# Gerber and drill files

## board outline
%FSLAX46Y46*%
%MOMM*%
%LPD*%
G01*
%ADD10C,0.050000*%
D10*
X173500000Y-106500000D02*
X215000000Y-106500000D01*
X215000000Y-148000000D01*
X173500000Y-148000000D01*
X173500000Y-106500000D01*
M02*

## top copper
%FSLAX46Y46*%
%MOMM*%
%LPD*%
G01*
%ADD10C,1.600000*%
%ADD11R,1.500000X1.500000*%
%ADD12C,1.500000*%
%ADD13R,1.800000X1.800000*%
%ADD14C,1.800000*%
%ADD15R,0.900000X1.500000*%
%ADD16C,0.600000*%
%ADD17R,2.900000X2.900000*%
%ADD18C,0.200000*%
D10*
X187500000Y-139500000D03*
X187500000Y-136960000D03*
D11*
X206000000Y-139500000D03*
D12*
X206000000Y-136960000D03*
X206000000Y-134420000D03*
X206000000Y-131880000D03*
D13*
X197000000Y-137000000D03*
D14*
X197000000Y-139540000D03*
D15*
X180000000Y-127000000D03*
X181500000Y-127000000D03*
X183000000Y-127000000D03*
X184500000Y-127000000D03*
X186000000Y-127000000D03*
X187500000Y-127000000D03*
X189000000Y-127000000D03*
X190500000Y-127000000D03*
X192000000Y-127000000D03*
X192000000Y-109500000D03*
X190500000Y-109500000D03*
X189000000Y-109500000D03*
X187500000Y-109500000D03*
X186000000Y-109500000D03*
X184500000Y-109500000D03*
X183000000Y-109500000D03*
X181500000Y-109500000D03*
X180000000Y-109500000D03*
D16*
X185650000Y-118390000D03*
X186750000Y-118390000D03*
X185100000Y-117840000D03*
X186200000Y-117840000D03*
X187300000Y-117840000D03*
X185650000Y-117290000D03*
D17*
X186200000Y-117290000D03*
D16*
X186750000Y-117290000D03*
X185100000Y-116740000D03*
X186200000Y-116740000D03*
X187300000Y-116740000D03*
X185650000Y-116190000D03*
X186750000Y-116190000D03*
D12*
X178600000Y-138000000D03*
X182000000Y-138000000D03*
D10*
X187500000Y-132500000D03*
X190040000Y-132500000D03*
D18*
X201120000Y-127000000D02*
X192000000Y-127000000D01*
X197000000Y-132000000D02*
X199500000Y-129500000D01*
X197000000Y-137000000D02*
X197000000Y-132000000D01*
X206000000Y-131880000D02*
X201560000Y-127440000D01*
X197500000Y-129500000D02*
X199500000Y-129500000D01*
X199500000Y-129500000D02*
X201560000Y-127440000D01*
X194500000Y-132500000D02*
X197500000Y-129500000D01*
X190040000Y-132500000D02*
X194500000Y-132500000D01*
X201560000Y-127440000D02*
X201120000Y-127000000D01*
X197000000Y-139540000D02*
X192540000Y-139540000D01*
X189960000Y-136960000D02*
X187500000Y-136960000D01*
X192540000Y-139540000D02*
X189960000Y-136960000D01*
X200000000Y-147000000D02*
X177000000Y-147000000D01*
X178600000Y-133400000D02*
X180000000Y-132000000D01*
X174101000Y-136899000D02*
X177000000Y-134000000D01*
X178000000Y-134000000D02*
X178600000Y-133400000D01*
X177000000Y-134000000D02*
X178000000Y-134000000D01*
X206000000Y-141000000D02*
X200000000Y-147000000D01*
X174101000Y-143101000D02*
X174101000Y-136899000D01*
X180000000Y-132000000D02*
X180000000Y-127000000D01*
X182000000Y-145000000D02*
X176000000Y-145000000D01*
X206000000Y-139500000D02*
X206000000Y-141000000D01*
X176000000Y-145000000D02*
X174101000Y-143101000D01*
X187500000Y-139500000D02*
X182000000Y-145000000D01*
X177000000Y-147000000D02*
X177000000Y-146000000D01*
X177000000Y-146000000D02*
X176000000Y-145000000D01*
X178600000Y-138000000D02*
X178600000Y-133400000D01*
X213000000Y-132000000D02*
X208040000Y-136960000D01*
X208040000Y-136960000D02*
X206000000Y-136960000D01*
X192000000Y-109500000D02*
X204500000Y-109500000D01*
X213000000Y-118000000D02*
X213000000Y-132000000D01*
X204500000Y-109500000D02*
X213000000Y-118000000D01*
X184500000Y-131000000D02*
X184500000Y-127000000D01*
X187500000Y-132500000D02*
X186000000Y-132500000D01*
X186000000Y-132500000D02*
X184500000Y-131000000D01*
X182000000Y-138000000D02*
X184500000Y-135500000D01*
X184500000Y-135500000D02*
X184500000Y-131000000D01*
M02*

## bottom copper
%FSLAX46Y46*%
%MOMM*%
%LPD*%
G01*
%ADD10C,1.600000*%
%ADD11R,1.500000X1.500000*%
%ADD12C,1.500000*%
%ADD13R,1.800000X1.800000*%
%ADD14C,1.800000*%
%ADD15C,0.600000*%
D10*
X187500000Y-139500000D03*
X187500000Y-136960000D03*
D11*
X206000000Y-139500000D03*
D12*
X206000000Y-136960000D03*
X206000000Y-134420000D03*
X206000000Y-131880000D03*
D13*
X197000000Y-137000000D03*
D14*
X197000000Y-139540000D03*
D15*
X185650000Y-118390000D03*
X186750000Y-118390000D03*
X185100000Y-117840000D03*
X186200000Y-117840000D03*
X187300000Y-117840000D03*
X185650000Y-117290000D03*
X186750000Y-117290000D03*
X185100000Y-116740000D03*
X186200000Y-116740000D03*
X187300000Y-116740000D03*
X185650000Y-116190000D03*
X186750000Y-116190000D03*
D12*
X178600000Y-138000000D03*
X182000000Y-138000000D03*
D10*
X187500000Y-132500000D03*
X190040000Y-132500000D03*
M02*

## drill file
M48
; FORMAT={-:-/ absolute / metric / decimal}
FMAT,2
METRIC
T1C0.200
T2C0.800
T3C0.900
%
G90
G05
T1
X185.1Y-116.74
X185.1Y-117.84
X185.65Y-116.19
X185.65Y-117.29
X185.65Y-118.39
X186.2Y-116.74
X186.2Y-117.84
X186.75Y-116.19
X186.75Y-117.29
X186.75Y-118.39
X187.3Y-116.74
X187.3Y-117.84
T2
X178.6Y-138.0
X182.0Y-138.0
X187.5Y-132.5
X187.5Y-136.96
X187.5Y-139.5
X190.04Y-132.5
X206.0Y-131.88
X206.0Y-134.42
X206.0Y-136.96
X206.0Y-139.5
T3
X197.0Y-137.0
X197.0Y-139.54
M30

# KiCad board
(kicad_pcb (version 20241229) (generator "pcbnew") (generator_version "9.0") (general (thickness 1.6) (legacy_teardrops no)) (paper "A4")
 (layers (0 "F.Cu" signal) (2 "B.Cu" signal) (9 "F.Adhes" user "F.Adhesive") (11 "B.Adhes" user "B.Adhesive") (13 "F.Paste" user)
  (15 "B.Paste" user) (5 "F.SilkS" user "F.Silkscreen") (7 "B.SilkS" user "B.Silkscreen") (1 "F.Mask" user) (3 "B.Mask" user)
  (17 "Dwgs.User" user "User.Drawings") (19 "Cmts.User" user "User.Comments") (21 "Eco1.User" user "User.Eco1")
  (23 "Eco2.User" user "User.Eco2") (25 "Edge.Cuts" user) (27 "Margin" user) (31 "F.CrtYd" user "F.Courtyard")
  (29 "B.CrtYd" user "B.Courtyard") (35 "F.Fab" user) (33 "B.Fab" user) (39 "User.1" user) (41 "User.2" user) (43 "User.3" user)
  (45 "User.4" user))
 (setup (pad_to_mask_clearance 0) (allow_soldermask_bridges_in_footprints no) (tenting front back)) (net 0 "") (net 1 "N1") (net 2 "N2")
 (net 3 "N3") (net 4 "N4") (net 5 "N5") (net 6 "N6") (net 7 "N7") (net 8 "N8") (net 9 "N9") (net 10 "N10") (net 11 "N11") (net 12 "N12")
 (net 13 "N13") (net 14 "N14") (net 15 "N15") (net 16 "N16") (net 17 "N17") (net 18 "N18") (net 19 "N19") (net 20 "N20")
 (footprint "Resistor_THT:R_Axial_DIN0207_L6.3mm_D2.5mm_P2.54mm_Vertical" (layer "F.Cu") (at 187.5 139.5 90)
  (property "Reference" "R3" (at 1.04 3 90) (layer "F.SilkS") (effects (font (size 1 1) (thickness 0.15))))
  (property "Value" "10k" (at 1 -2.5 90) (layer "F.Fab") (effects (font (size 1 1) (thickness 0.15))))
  (pad "1" thru_hole circle (at 0 0 90) (size 1.6 1.6) (drill 0.8) (layers "*.Cu" "*.Mask") (remove_unused_layers no) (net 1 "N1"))
  (pad "2" thru_hole circle (at 2.54 0 90) (size 1.6 1.6) (drill 0.8) (layers "*.Cu" "*.Mask") (remove_unused_layers no) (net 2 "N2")))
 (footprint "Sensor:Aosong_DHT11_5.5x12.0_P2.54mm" (layer "F.Cu") (at 206 139.5 180)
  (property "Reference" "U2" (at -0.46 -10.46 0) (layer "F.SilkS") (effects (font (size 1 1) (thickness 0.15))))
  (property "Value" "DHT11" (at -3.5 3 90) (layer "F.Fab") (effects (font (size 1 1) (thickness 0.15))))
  (pad "1" thru_hole rect (at 0 0 180) (size 1.5 1.5) (drill 0.8) (layers "*.Cu" "*.Mask") (remove_unused_layers no) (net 1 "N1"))
  (pad "2" thru_hole circle (at 0 2.54 180) (size 1.5 1.5) (drill 0.8) (layers "*.Cu" "*.Mask") (remove_unused_layers no) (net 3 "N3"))
  (pad "3" thru_hole circle (at 0 5.08 180) (size 1.5 1.5) (drill 0.8) (layers "*.Cu" "*.Mask") (remove_unused_layers no) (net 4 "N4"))
  (pad "4" thru_hole circle (at 0 7.62 180) (size 1.5 1.5) (drill 0.8) (layers "*.Cu" "*.Mask") (remove_unused_layers no) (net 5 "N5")))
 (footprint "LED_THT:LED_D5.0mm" (layer "F.Cu") (at 197 137 -90)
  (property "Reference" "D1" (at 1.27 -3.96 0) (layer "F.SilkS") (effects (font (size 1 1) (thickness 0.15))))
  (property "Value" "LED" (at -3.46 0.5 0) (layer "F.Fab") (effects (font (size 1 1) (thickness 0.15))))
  (pad "1" thru_hole rect (at 0 0 270) (size 1.8 1.8) (drill 0.9) (layers "*.Cu" "*.Mask") (remove_unused_layers no) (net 5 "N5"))
  (pad "2" thru_hole circle (at 2.54 0 270) (size 1.8 1.8) (drill 0.9) (layers "*.Cu" "*.Mask") (remove_unused_layers no) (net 2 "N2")))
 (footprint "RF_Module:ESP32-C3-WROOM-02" (layer "F.Cu") (at 186 118.25 90)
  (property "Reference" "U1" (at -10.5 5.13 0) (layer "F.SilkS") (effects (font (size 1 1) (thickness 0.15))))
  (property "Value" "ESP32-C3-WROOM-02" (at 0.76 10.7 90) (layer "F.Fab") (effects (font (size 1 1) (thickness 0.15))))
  (pad "" smd rect (at -0.14 -0.9 90) (size 0.7 0.7) (layers "F.Paste"))
  (pad "" smd rect (at -0.14 0.2 90) (size 0.7 0.7) (layers "F.Paste"))
  (pad "" smd rect (at -0.14 1.3 90) (size 0.7 0.7) (layers "F.Paste"))
  (pad "" smd rect (at 0.96 -0.9 90) (size 0.7 0.7) (layers "F.Paste"))
  (pad "" smd rect (at 0.96 0.2 90) (size 0.7 0.7) (layers "F.Paste"))
  (pad "" smd rect (at 0.96 1.3 90) (size 0.7 0.7) (layers "F.Paste"))
  (pad "" smd rect (at 2.06 -0.9 90) (size 0.7 0.7) (layers "F.Paste"))
  (pad "" smd rect (at 2.06 0.2 90) (size 0.7 0.7) (layers "F.Paste"))
  (pad "" smd rect (at 2.06 1.3 90) (size 0.7 0.7) (layers "F.Paste"))
  (pad "1" smd rect (at -8.75 -6 90) (size 1.5 0.9) (layers "F.Cu" "F.Mask" "F.Paste") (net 1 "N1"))
  (pad "2" smd rect (at -8.75 -4.5 90) (size 1.5 0.9) (layers "F.Cu" "F.Mask" "F.Paste") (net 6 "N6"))
  (pad "3" smd rect (at -8.75 -3 90) (size 1.5 0.9) (layers "F.Cu" "F.Mask" "F.Paste") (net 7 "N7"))
  (pad "4" smd rect (at -8.75 -1.5 90) (size 1.5 0.9) (layers "F.Cu" "F.Mask" "F.Paste") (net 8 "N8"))
  (pad "5" smd rect (at -8.75 0 90) (size 1.5 0.9) (layers "F.Cu" "F.Mask" "F.Paste") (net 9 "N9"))
  (pad "6" smd rect (at -8.75 1.5 90) (size 1.5 0.9) (layers "F.Cu" "F.Mask" "F.Paste") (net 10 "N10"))
  (pad "7" smd rect (at -8.75 3 90) (size 1.5 0.9) (layers "F.Cu" "F.Mask" "F.Paste") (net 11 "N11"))
  (pad "8" smd rect (at -8.75 4.5 90) (size 1.5 0.9) (layers "F.Cu" "F.Mask" "F.Paste") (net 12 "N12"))
  (pad "9" smd rect (at -8.75 6 90) (size 1.5 0.9) (layers "F.Cu" "F.Mask" "F.Paste") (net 5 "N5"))
  (pad "10" smd rect (at 8.75 6 90) (size 1.5 0.9) (layers "F.Cu" "F.Mask" "F.Paste") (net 3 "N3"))
  (pad "11" smd rect (at 8.75 4.5 90) (size 1.5 0.9) (layers "F.Cu" "F.Mask" "F.Paste") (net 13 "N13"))
  (pad "12" smd rect (at 8.75 3 90) (size 1.5 0.9) (layers "F.Cu" "F.Mask" "F.Paste") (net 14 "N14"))
  (pad "13" smd rect (at 8.75 1.5 90) (size 1.5 0.9) (layers "F.Cu" "F.Mask" "F.Paste") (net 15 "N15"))
  (pad "14" smd rect (at 8.75 0 90) (size 1.5 0.9) (layers "F.Cu" "F.Mask" "F.Paste") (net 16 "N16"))
  (pad "15" smd rect (at 8.75 -1.5 90) (size 1.5 0.9) (layers "F.Cu" "F.Mask" "F.Paste") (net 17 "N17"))
  (pad "16" smd rect (at 8.75 -3 90) (size 1.5 0.9) (layers "F.Cu" "F.Mask" "F.Paste") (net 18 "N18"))
  (pad "17" smd rect (at 8.75 -4.5 90) (size 1.5 0.9) (layers "F.Cu" "F.Mask" "F.Paste") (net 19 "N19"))
  (pad "18" smd rect (at 8.75 -6 90) (size 1.5 0.9) (layers "F.Cu" "F.Mask" "F.Paste") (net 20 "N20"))
  (pad "19" thru_hole circle (at -0.14 -0.35 90) (size 0.6 0.6) (drill 0.2) (layers "*.Cu" "F.Mask") (remove_unused_layers no) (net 5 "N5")
   (zone_connect 2))
  (pad "19" thru_hole circle (at -0.14 0.75 90) (size 0.6 0.6) (drill 0.2) (layers "*.Cu" "F.Mask") (remove_unused_layers no) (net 5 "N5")
   (zone_connect 2))
  (pad "19" thru_hole circle (at 0.41 -0.9 90) (size 0.6 0.6) (drill 0.2) (layers "*.Cu" "F.Mask") (remove_unused_layers no) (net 5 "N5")
   (zone_connect 2))
  (pad "19" thru_hole circle (at 0.41 0.2 90) (size 0.6 0.6) (drill 0.2) (layers "*.Cu" "F.Mask") (remove_unused_layers no) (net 5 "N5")
   (zone_connect 2))
  (pad "19" thru_hole circle (at 0.41 1.3 90) (size 0.6 0.6) (drill 0.2) (layers "*.Cu" "F.Mask") (remove_unused_layers no) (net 5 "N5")
   (zone_connect 2))
  (pad "19" thru_hole circle (at 0.96 -0.35 90) (size 0.6 0.6) (drill 0.2) (layers "*.Cu" "F.Mask") (remove_unused_layers no) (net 5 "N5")
   (zone_connect 2))
  (pad "19" smd rect (at 0.96 0.2 90) (size 2.9 2.9) (layers "F.Cu" "F.Mask") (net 5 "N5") (zone_connect 2))
  (pad "19" thru_hole circle (at 0.96 0.75 90) (size 0.6 0.6) (drill 0.2) (layers "*.Cu" "F.Mask") (remove_unused_layers no) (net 5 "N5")
   (zone_connect 2))
  (pad "19" thru_hole circle (at 1.51 -0.9 90) (size 0.6 0.6) (drill 0.2) (layers "*.Cu" "F.Mask") (remove_unused_layers no) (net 5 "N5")
   (zone_connect 2))
  (pad "19" thru_hole circle (at 1.51 0.2 90) (size 0.6 0.6) (drill 0.2) (layers "*.Cu" "F.Mask") (remove_unused_layers no) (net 5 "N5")
   (zone_connect 2))
  (pad "19" thru_hole circle (at 1.51 1.3 90) (size 0.6 0.6) (drill 0.2) (layers "*.Cu" "F.Mask") (remove_unused_layers no) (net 5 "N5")
   (zone_connect 2))
  (pad "19" thru_hole circle (at 2.06 -0.35 90) (size 0.6 0.6) (drill 0.2) (layers "*.Cu" "F.Mask") (remove_unused_layers no) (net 5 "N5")
   (zone_connect 2))
  (pad "19" thru_hole circle (at 2.06 0.75 90) (size 0.6 0.6) (drill 0.2) (layers "*.Cu" "F.Mask") (remove_unused_layers no) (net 5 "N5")
   (zone_connect 2))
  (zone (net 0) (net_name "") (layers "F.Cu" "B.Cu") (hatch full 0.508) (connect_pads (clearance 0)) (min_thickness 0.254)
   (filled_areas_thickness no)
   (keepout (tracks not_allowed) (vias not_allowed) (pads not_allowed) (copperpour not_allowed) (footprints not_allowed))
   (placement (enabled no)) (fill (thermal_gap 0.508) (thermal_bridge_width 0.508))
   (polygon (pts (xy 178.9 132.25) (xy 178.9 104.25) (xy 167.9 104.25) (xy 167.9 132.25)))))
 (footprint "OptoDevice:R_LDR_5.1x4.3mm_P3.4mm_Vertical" (layer "F.Cu") (at 178.6 138)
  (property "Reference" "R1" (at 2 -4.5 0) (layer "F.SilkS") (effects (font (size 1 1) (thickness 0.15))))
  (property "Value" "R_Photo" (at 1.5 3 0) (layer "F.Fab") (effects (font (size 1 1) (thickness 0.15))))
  (pad "1" thru_hole circle (at 0 0) (size 1.5 1.5) (drill 0.8) (layers "*.Cu" "*.Mask") (remove_unused_layers no) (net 1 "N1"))
  (pad "2" thru_hole circle (at 3.4 0) (size 1.5 1.5) (drill 0.8) (layers "*.Cu" "*.Mask") (remove_unused_layers no) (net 8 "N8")))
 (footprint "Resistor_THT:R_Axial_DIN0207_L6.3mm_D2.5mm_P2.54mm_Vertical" (layer "F.Cu") (at 187.5 132.5)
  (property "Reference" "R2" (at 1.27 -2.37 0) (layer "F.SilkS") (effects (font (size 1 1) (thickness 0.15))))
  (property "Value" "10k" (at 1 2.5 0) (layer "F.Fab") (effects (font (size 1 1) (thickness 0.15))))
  (pad "1" thru_hole circle (at 0 0) (size 1.6 1.6) (drill 0.8) (layers "*.Cu" "*.Mask") (remove_unused_layers no) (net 8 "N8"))
  (pad "2" thru_hole circle (at 2.54 0) (size 1.6 1.6) (drill 0.8) (layers "*.Cu" "*.Mask") (remove_unused_layers no) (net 5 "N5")))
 (gr_rect (start 173.5 106.5) (end 215 148) (stroke (width 0.05) (type default)) (fill no) (layer "Edge.Cuts"))
 (segment (start 201.12 127) (end 192 127) (width 0.2) (layer "F.Cu") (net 5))
 (segment (start 197 132) (end 199.5 129.5) (width 0.2) (layer "F.Cu") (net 5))
 (segment (start 197 137) (end 197 132) (width 0.2) (layer "F.Cu") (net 5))
 (segment (start 206 131.88) (end 201.56 127.44) (width 0.2) (layer "F.Cu") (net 5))
 (segment (start 197.5 129.5) (end 199.5 129.5) (width 0.2) (layer "F.Cu") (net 5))
 (segment (start 199.5 129.5) (end 201.56 127.44) (width 0.2) (layer "F.Cu") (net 5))
 (segment (start 194.5 132.5) (end 197.5 129.5) (width 0.2) (layer "F.Cu") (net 5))
 (segment (start 190.04 132.5) (end 194.5 132.5) (width 0.2) (layer "F.Cu") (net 5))
 (segment (start 201.56 127.44) (end 201.12 127) (width 0.2) (layer "F.Cu") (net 5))
 (segment (start 197 139.54) (end 192.54 139.54) (width 0.2) (layer "F.Cu") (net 2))
 (segment (start 189.96 136.96) (end 187.5 136.96) (width 0.2) (layer "F.Cu") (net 2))
 (segment (start 192.54 139.54) (end 189.96 136.96) (width 0.2) (layer "F.Cu") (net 2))
 (segment (start 200 147) (end 177 147) (width 0.2) (layer "F.Cu") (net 1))
 (segment (start 178.6 133.4) (end 180 132) (width 0.2) (layer "F.Cu") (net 1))
 (segment (start 174.101 136.899) (end 177 134) (width 0.2) (layer "F.Cu") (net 1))
 (segment (start 178 134) (end 178.6 133.4) (width 0.2) (layer "F.Cu") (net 1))
 (segment (start 177 134) (end 178 134) (width 0.2) (layer "F.Cu") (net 1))
 (segment (start 206 141) (end 200 147) (width 0.2) (layer "F.Cu") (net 1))
 (segment (start 174.101 143.101) (end 174.101 136.899) (width 0.2) (layer "F.Cu") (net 1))
 (segment (start 180 132) (end 180 127) (width 0.2) (layer "F.Cu") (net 1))
 (segment (start 182 145) (end 176 145) (width 0.2) (layer "F.Cu") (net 1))
 (segment (start 206 139.5) (end 206 141) (width 0.2) (layer "F.Cu") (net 1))
 (segment (start 176 145) (end 174.101 143.101) (width 0.2) (layer "F.Cu") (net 1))
 (segment (start 187.5 139.5) (end 182 145) (width 0.2) (layer "F.Cu") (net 1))
 (segment (start 177 147) (end 177 146) (width 0.2) (layer "F.Cu") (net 1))
 (segment (start 177 146) (end 176 145) (width 0.2) (layer "F.Cu") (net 1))
 (segment (start 178.6 138) (end 178.6 133.4) (width 0.2) (layer "F.Cu") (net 1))
 (segment (start 213 132) (end 208.04 136.96) (width 0.2) (layer "F.Cu") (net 3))
 (segment (start 208.04 136.96) (end 206 136.96) (width 0.2) (layer "F.Cu") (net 3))
 (segment (start 192 109.5) (end 204.5 109.5) (width 0.2) (layer "F.Cu") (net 3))
 (segment (start 213 118) (end 213 132) (width 0.2) (layer "F.Cu") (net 3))
 (segment (start 204.5 109.5) (end 213 118) (width 0.2) (layer "F.Cu") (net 3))
 (segment (start 184.5 131) (end 184.5 127) (width 0.2) (layer "F.Cu") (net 8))
 (segment (start 187.5 132.5) (end 186 132.5) (width 0.2) (layer "F.Cu") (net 8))
 (segment (start 186 132.5) (end 184.5 131) (width 0.2) (layer "F.Cu") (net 8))
 (segment (start 182 138) (end 184.5 135.5) (width 0.2) (layer "F.Cu") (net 8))
 (segment (start 184.5 135.5) (end 184.5 131) (width 0.2) (layer "F.Cu") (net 8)))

